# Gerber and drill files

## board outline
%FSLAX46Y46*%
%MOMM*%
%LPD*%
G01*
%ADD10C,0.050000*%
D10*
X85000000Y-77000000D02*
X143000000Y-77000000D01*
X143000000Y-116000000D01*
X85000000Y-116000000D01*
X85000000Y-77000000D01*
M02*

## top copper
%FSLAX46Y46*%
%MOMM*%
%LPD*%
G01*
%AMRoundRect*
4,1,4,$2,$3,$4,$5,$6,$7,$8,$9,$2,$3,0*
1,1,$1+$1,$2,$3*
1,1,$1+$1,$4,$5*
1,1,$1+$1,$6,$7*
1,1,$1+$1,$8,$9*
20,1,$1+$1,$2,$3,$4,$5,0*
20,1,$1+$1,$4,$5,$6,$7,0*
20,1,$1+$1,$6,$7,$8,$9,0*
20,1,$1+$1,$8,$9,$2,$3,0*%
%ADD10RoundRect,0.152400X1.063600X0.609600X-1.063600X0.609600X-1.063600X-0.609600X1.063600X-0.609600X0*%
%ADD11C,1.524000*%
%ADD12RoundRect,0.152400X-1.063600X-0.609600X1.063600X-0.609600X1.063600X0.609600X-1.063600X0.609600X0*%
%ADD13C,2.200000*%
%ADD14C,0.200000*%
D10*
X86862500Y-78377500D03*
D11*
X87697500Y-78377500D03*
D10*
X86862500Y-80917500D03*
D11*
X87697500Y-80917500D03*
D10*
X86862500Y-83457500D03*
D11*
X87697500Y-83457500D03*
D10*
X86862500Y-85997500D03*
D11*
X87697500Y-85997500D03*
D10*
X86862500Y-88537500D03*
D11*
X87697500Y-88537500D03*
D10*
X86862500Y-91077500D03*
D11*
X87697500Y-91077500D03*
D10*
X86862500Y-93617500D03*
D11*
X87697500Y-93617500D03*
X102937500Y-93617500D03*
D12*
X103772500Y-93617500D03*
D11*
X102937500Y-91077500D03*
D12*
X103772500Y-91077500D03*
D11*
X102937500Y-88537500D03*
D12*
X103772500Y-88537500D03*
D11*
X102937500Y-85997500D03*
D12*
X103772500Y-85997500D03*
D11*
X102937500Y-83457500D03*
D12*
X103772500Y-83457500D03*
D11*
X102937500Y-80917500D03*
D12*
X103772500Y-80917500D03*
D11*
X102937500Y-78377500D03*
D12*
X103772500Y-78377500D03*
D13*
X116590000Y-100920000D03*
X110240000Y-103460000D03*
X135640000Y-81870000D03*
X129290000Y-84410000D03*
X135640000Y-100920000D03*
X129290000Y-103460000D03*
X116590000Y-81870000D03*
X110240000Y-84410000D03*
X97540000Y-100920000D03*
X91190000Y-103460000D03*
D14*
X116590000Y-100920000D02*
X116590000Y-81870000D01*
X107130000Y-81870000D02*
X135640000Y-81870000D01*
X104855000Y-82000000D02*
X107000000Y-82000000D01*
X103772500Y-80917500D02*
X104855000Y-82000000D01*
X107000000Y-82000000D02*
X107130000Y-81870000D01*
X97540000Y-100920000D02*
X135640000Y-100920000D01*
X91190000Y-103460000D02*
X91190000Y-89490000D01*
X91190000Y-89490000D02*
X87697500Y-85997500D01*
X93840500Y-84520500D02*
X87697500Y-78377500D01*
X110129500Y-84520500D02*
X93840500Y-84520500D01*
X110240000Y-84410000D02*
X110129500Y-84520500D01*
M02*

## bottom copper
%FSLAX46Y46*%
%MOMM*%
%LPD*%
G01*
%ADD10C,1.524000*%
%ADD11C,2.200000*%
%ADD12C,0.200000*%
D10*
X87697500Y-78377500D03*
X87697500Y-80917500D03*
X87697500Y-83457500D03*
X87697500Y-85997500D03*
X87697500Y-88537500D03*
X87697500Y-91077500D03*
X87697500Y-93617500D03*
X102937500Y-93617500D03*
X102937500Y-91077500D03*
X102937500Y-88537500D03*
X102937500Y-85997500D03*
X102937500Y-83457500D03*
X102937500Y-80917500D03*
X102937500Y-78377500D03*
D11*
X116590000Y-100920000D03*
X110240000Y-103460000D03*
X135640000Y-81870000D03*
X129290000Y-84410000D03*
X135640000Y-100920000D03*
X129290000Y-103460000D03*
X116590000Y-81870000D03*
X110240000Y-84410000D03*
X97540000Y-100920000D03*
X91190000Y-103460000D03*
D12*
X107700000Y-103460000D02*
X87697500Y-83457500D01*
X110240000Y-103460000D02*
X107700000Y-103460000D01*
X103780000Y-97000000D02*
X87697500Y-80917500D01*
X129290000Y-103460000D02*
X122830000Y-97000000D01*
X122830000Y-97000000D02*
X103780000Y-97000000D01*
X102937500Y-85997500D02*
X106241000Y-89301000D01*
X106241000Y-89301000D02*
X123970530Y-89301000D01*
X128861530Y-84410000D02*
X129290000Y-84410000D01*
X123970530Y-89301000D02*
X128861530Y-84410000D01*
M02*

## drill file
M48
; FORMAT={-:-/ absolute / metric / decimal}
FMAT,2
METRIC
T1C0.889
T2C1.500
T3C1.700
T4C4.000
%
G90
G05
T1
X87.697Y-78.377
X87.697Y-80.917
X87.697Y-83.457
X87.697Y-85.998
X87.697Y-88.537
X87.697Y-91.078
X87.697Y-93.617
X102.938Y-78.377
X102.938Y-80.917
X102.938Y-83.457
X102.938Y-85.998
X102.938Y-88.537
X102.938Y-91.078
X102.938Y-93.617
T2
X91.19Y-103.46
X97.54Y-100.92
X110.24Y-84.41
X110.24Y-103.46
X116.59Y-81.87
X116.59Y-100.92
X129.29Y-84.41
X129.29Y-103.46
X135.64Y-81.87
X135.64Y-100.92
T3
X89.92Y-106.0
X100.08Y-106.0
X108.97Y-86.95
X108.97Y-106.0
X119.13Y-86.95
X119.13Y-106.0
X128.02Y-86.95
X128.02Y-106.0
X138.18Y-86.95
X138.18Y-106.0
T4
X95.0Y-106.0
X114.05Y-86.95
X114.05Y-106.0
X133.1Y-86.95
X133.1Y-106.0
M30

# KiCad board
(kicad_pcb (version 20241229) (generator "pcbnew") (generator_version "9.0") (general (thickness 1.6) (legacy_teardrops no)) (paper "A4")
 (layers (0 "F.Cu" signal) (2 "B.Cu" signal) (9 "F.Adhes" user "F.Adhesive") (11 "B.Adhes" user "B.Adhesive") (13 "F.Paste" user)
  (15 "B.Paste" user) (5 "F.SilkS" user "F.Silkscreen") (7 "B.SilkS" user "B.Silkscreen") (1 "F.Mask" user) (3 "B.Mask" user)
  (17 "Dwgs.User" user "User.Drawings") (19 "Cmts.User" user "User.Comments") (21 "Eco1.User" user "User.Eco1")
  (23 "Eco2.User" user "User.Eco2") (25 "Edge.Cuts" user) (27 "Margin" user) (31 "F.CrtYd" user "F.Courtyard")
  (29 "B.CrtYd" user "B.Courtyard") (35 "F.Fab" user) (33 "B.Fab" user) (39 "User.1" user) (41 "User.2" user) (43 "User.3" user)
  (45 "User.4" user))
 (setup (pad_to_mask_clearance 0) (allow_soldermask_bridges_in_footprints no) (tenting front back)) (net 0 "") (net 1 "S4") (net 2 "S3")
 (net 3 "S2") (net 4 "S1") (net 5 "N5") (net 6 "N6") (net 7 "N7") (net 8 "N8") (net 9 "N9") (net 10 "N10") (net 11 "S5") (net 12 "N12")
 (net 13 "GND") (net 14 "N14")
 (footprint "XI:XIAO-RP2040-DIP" (layer "F.Cu") (at 95.3175 85.9975)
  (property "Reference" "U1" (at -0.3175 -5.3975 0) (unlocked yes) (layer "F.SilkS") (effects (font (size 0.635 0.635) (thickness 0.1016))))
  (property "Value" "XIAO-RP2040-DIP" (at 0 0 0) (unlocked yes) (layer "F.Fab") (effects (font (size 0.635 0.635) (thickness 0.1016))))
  (pad "1" smd roundrect (at -8.455 -7.62 180) (size 2.432 1.524) (layers "F.Cu" "F.Mask") (roundrect_rratio 0.1) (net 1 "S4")
   (thermal_bridge_angle 45))
  (pad "1" thru_hole circle (at -7.62 -7.62 180) (size 1.524 1.524) (drill 0.889) (layers "*.Cu" "*.Mask") (remove_unused_layers no)
   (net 1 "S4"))
  (pad "2" smd roundrect (at -8.455 -5.08 180) (size 2.432 1.524) (layers "F.Cu" "F.Mask") (roundrect_rratio 0.1) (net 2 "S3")
   (thermal_bridge_angle 45))
  (pad "2" thru_hole circle (at -7.62 -5.08 180) (size 1.524 1.524) (drill 0.889) (layers "*.Cu" "*.Mask") (remove_unused_layers no)
   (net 2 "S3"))
  (pad "3" smd roundrect (at -8.455 -2.54 180) (size 2.432 1.524) (layers "F.Cu" "F.Mask") (roundrect_rratio 0.1) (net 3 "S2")
   (thermal_bridge_angle 45))
  (pad "3" thru_hole circle (at -7.62 -2.54 180) (size 1.524 1.524) (drill 0.889) (layers "*.Cu" "*.Mask") (remove_unused_layers no)
   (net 3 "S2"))
  (pad "4" smd roundrect (at -8.455 0 180) (size 2.432 1.524) (layers "F.Cu" "F.Mask") (roundrect_rratio 0.1) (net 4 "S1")
   (thermal_bridge_angle 45))
  (pad "4" thru_hole circle (at -7.62 0 180) (size 1.524 1.524) (drill 0.889) (layers "*.Cu" "*.Mask") (remove_unused_layers no)
   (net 4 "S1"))
  (pad "5" smd roundrect (at -8.455 2.54 180) (size 2.432 1.524) (layers "F.Cu" "F.Mask") (roundrect_rratio 0.1) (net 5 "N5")
   (thermal_bridge_angle 45))
  (pad "5" thru_hole circle (at -7.62 2.54 180) (size 1.524 1.524) (drill 0.889) (layers "*.Cu" "*.Mask") (remove_unused_layers no)
   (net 5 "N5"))
  (pad "6" smd roundrect (at -8.455 5.08 180) (size 2.432 1.524) (layers "F.Cu" "F.Mask") (roundrect_rratio 0.1) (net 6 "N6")
   (thermal_bridge_angle 45))
  (pad "6" thru_hole circle (at -7.62 5.08 180) (size 1.524 1.524) (drill 0.889) (layers "*.Cu" "*.Mask") (remove_unused_layers no)
   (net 6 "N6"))
  (pad "7" smd roundrect (at -8.455 7.62 180) (size 2.432 1.524) (layers "F.Cu" "F.Mask") (roundrect_rratio 0.1) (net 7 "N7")
   (thermal_bridge_angle 45))
  (pad "7" thru_hole circle (at -7.62 7.62 180) (size 1.524 1.524) (drill 0.889) (layers "*.Cu" "*.Mask") (remove_unused_layers no)
   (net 7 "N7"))
  (pad "8" thru_hole circle (at 7.62 7.62) (size 1.524 1.524) (drill 0.889) (layers "*.Cu" "*.Mask") (remove_unused_layers no) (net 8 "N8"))
  (pad "8" smd roundrect (at 8.455 7.62) (size 2.432 1.524) (layers "F.Cu" "F.Mask") (roundrect_rratio 0.1) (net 8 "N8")
   (thermal_bridge_angle 45))
  (pad "9" thru_hole circle (at 7.62 5.08) (size 1.524 1.524) (drill 0.889) (layers "*.Cu" "*.Mask") (remove_unused_layers no) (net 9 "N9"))
  (pad "9" smd roundrect (at 8.455 5.08) (size 2.432 1.524) (layers "F.Cu" "F.Mask") (roundrect_rratio 0.1) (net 9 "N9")
   (thermal_bridge_angle 45))
  (pad "10" thru_hole circle (at 7.62 2.54) (size 1.524 1.524) (drill 0.889) (layers "*.Cu" "*.Mask") (remove_unused_layers no)
   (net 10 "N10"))
  (pad "10" smd roundrect (at 8.455 2.54) (size 2.432 1.524) (layers "F.Cu" "F.Mask") (roundrect_rratio 0.1) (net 10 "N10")
   (thermal_bridge_angle 45))
  (pad "11" thru_hole circle (at 7.62 0) (size 1.524 1.524) (drill 0.889) (layers "*.Cu" "*.Mask") (remove_unused_layers no) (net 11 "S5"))
  (pad "11" smd roundrect (at 8.455 0) (size 2.432 1.524) (layers "F.Cu" "F.Mask") (roundrect_rratio 0.1) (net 11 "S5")
   (thermal_bridge_angle 45))
  (pad "12" thru_hole circle (at 7.62 -2.54) (size 1.524 1.524) (drill 0.889) (layers "*.Cu" "*.Mask") (remove_unused_layers no)
   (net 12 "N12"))
  (pad "12" smd roundrect (at 8.455 -2.54) (size 2.432 1.524) (layers "F.Cu" "F.Mask") (roundrect_rratio 0.1) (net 12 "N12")
   (thermal_bridge_angle 45))
  (pad "13" thru_hole circle (at 7.62 -5.08) (size 1.524 1.524) (drill 0.889) (layers "*.Cu" "*.Mask") (remove_unused_layers no)
   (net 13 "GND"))
  (pad "13" smd roundrect (at 8.455 -5.08) (size 2.432 1.524) (layers "F.Cu" "F.Mask") (roundrect_rratio 0.1) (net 13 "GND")
   (thermal_bridge_angle 45))
  (pad "14" thru_hole circle (at 7.62 -7.62) (size 1.524 1.524) (drill 0.889) (layers "*.Cu" "*.Mask") (remove_unused_layers no)
   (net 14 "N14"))
  (pad "14" smd roundrect (at 8.455 -7.62) (size 2.432 1.524) (layers "F.Cu" "F.Mask") (roundrect_rratio 0.1) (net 14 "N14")
   (thermal_bridge_angle 45)))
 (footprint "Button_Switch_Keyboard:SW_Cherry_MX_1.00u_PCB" (layer "F.Cu") (at 116.59 100.92)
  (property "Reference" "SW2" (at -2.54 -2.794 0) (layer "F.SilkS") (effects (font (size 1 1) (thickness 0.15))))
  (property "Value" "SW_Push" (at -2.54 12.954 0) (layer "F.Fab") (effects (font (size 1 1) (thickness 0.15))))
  (pad "" np_thru_hole circle (at -7.62 5.08) (size 1.7 1.7) (drill 1.7) (layers "*.Cu" "*.Mask"))
  (pad "" np_thru_hole circle (at -2.54 5.08) (size 4 4) (drill 4) (layers "*.Cu" "*.Mask"))
  (pad "" np_thru_hole circle (at 2.54 5.08) (size 1.7 1.7) (drill 1.7) (layers "*.Cu" "*.Mask"))
  (pad "1" thru_hole circle (at 0 0) (size 2.2 2.2) (drill 1.5) (layers "*.Cu" "*.Mask") (remove_unused_layers no) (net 13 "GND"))
  (pad "2" thru_hole circle (at -6.35 2.54) (size 2.2 2.2) (drill 1.5) (layers "*.Cu" "*.Mask") (remove_unused_layers no) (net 3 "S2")))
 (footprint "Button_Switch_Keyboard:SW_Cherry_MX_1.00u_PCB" (layer "F.Cu") (at 135.64 81.87)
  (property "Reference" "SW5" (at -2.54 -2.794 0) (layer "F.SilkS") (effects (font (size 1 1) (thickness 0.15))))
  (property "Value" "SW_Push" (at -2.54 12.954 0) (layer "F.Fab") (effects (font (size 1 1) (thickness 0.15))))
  (pad "" np_thru_hole circle (at -7.62 5.08) (size 1.7 1.7) (drill 1.7) (layers "*.Cu" "*.Mask"))
  (pad "" np_thru_hole circle (at -2.54 5.08) (size 4 4) (drill 4) (layers "*.Cu" "*.Mask"))
  (pad "" np_thru_hole circle (at 2.54 5.08) (size 1.7 1.7) (drill 1.7) (layers "*.Cu" "*.Mask"))
  (pad "1" thru_hole circle (at 0 0) (size 2.2 2.2) (drill 1.5) (layers "*.Cu" "*.Mask") (remove_unused_layers no) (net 13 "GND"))
  (pad "2" thru_hole circle (at -6.35 2.54) (size 2.2 2.2) (drill 1.5) (layers "*.Cu" "*.Mask") (remove_unused_layers no) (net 11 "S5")))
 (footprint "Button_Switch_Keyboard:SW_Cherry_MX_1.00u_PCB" (layer "F.Cu") (at 135.64 100.92)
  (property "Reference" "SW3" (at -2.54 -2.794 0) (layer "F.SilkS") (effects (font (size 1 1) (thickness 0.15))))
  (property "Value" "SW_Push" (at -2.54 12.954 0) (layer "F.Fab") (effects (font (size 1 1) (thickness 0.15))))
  (pad "" np_thru_hole circle (at -7.62 5.08) (size 1.7 1.7) (drill 1.7) (layers "*.Cu" "*.Mask"))
  (pad "" np_thru_hole circle (at -2.54 5.08) (size 4 4) (drill 4) (layers "*.Cu" "*.Mask"))
  (pad "" np_thru_hole circle (at 2.54 5.08) (size 1.7 1.7) (drill 1.7) (layers "*.Cu" "*.Mask"))
  (pad "1" thru_hole circle (at 0 0) (size 2.2 2.2) (drill 1.5) (layers "*.Cu" "*.Mask") (remove_unused_layers no) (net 13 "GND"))
  (pad "2" thru_hole circle (at -6.35 2.54) (size 2.2 2.2) (drill 1.5) (layers "*.Cu" "*.Mask") (remove_unused_layers no) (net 2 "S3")))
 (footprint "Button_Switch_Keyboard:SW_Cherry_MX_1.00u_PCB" (layer "F.Cu") (at 116.59 81.87)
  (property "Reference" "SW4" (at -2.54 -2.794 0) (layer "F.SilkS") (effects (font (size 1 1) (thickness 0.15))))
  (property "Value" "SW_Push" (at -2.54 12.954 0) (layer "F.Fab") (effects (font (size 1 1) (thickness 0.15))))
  (pad "" np_thru_hole circle (at -7.62 5.08) (size 1.7 1.7) (drill 1.7) (layers "*.Cu" "*.Mask"))
  (pad "" np_thru_hole circle (at -2.54 5.08) (size 4 4) (drill 4) (layers "*.Cu" "*.Mask"))
  (pad "" np_thru_hole circle (at 2.54 5.08) (size 1.7 1.7) (drill 1.7) (layers "*.Cu" "*.Mask"))
  (pad "1" thru_hole circle (at 0 0) (size 2.2 2.2) (drill 1.5) (layers "*.Cu" "*.Mask") (remove_unused_layers no) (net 13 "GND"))
  (pad "2" thru_hole circle (at -6.35 2.54) (size 2.2 2.2) (drill 1.5) (layers "*.Cu" "*.Mask") (remove_unused_layers no) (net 1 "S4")))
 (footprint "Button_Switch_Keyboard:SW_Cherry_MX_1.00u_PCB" (layer "F.Cu") (at 97.54 100.92)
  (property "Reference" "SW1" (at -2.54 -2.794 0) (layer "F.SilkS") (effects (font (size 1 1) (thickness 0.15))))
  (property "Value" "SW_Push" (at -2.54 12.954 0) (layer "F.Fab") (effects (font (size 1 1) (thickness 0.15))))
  (pad "" np_thru_hole circle (at -7.62 5.08) (size 1.7 1.7) (drill 1.7) (layers "*.Cu" "*.Mask"))
  (pad "" np_thru_hole circle (at -2.54 5.08) (size 4 4) (drill 4) (layers "*.Cu" "*.Mask"))
  (pad "" np_thru_hole circle (at 2.54 5.08) (size 1.7 1.7) (drill 1.7) (layers "*.Cu" "*.Mask"))
  (pad "1" thru_hole circle (at 0 0) (size 2.2 2.2) (drill 1.5) (layers "*.Cu" "*.Mask") (remove_unused_layers no) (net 13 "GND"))
  (pad "2" thru_hole circle (at -6.35 2.54) (size 2.2 2.2) (drill 1.5) (layers "*.Cu" "*.Mask") (remove_unused_layers no) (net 4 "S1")))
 (gr_rect (start 85 77) (end 143 116) (stroke (width 0.05) (type default)) (fill no) (layer "Edge.Cuts"))
 (segment (start 116.59 100.92) (end 116.59 81.87) (width 0.2) (layer "F.Cu") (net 13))
 (segment (start 107.13 81.87) (end 135.64 81.87) (width 0.2) (layer "F.Cu") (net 13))
 (segment (start 104.855 82) (end 107 82) (width 0.2) (layer "F.Cu") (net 13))
 (segment (start 103.7725 80.9175) (end 104.855 82) (width 0.2) (layer "F.Cu") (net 13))
 (segment (start 107 82) (end 107.13 81.87) (width 0.2) (layer "F.Cu") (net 13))
 (segment (start 97.54 100.92) (end 135.64 100.92) (width 0.2) (layer "F.Cu") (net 13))
 (segment (start 91.19 103.46) (end 91.19 89.49) (width 0.2) (layer "F.Cu") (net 4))
 (segment (start 91.19 89.49) (end 87.6975 85.9975) (width 0.2) (layer "F.Cu") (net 4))
 (segment (start 107.7 103.46) (end 87.6975 83.4575) (width 0.2) (layer "B.Cu") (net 3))
 (segment (start 110.24 103.46) (end 107.7 103.46) (width 0.2) (layer "B.Cu") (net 3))
 (segment (start 103.78 97) (end 87.6975 80.9175) (width 0.2) (layer "B.Cu") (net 2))
 (segment (start 129.29 103.46) (end 122.83 97) (width 0.2) (layer "B.Cu") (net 2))
 (segment (start 122.83 97) (end 103.78 97) (width 0.2) (layer "B.Cu") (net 2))
 (segment (start 93.8405 84.5205) (end 87.6975 78.3775) (width 0.2) (layer "F.Cu") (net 1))
 (segment (start 110.1295 84.5205) (end 93.8405 84.5205) (width 0.2) (layer "F.Cu") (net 1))
 (segment (start 110.24 84.41) (end 110.1295 84.5205) (width 0.2) (layer "F.Cu") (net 1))
 (segment (start 102.9375 85.9975) (end 106.241 89.301) (width 0.2) (layer "B.Cu") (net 11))
 (segment (start 106.241 89.301) (end 123.97053 89.301) (width 0.2) (layer "B.Cu") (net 11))
 (segment (start 128.86153 84.41) (end 129.29 84.41) (width 0.2) (layer "B.Cu") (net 11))
 (segment (start 123.97053 89.301) (end 128.86153 84.41) (width 0.2) (layer "B.Cu") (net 11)))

